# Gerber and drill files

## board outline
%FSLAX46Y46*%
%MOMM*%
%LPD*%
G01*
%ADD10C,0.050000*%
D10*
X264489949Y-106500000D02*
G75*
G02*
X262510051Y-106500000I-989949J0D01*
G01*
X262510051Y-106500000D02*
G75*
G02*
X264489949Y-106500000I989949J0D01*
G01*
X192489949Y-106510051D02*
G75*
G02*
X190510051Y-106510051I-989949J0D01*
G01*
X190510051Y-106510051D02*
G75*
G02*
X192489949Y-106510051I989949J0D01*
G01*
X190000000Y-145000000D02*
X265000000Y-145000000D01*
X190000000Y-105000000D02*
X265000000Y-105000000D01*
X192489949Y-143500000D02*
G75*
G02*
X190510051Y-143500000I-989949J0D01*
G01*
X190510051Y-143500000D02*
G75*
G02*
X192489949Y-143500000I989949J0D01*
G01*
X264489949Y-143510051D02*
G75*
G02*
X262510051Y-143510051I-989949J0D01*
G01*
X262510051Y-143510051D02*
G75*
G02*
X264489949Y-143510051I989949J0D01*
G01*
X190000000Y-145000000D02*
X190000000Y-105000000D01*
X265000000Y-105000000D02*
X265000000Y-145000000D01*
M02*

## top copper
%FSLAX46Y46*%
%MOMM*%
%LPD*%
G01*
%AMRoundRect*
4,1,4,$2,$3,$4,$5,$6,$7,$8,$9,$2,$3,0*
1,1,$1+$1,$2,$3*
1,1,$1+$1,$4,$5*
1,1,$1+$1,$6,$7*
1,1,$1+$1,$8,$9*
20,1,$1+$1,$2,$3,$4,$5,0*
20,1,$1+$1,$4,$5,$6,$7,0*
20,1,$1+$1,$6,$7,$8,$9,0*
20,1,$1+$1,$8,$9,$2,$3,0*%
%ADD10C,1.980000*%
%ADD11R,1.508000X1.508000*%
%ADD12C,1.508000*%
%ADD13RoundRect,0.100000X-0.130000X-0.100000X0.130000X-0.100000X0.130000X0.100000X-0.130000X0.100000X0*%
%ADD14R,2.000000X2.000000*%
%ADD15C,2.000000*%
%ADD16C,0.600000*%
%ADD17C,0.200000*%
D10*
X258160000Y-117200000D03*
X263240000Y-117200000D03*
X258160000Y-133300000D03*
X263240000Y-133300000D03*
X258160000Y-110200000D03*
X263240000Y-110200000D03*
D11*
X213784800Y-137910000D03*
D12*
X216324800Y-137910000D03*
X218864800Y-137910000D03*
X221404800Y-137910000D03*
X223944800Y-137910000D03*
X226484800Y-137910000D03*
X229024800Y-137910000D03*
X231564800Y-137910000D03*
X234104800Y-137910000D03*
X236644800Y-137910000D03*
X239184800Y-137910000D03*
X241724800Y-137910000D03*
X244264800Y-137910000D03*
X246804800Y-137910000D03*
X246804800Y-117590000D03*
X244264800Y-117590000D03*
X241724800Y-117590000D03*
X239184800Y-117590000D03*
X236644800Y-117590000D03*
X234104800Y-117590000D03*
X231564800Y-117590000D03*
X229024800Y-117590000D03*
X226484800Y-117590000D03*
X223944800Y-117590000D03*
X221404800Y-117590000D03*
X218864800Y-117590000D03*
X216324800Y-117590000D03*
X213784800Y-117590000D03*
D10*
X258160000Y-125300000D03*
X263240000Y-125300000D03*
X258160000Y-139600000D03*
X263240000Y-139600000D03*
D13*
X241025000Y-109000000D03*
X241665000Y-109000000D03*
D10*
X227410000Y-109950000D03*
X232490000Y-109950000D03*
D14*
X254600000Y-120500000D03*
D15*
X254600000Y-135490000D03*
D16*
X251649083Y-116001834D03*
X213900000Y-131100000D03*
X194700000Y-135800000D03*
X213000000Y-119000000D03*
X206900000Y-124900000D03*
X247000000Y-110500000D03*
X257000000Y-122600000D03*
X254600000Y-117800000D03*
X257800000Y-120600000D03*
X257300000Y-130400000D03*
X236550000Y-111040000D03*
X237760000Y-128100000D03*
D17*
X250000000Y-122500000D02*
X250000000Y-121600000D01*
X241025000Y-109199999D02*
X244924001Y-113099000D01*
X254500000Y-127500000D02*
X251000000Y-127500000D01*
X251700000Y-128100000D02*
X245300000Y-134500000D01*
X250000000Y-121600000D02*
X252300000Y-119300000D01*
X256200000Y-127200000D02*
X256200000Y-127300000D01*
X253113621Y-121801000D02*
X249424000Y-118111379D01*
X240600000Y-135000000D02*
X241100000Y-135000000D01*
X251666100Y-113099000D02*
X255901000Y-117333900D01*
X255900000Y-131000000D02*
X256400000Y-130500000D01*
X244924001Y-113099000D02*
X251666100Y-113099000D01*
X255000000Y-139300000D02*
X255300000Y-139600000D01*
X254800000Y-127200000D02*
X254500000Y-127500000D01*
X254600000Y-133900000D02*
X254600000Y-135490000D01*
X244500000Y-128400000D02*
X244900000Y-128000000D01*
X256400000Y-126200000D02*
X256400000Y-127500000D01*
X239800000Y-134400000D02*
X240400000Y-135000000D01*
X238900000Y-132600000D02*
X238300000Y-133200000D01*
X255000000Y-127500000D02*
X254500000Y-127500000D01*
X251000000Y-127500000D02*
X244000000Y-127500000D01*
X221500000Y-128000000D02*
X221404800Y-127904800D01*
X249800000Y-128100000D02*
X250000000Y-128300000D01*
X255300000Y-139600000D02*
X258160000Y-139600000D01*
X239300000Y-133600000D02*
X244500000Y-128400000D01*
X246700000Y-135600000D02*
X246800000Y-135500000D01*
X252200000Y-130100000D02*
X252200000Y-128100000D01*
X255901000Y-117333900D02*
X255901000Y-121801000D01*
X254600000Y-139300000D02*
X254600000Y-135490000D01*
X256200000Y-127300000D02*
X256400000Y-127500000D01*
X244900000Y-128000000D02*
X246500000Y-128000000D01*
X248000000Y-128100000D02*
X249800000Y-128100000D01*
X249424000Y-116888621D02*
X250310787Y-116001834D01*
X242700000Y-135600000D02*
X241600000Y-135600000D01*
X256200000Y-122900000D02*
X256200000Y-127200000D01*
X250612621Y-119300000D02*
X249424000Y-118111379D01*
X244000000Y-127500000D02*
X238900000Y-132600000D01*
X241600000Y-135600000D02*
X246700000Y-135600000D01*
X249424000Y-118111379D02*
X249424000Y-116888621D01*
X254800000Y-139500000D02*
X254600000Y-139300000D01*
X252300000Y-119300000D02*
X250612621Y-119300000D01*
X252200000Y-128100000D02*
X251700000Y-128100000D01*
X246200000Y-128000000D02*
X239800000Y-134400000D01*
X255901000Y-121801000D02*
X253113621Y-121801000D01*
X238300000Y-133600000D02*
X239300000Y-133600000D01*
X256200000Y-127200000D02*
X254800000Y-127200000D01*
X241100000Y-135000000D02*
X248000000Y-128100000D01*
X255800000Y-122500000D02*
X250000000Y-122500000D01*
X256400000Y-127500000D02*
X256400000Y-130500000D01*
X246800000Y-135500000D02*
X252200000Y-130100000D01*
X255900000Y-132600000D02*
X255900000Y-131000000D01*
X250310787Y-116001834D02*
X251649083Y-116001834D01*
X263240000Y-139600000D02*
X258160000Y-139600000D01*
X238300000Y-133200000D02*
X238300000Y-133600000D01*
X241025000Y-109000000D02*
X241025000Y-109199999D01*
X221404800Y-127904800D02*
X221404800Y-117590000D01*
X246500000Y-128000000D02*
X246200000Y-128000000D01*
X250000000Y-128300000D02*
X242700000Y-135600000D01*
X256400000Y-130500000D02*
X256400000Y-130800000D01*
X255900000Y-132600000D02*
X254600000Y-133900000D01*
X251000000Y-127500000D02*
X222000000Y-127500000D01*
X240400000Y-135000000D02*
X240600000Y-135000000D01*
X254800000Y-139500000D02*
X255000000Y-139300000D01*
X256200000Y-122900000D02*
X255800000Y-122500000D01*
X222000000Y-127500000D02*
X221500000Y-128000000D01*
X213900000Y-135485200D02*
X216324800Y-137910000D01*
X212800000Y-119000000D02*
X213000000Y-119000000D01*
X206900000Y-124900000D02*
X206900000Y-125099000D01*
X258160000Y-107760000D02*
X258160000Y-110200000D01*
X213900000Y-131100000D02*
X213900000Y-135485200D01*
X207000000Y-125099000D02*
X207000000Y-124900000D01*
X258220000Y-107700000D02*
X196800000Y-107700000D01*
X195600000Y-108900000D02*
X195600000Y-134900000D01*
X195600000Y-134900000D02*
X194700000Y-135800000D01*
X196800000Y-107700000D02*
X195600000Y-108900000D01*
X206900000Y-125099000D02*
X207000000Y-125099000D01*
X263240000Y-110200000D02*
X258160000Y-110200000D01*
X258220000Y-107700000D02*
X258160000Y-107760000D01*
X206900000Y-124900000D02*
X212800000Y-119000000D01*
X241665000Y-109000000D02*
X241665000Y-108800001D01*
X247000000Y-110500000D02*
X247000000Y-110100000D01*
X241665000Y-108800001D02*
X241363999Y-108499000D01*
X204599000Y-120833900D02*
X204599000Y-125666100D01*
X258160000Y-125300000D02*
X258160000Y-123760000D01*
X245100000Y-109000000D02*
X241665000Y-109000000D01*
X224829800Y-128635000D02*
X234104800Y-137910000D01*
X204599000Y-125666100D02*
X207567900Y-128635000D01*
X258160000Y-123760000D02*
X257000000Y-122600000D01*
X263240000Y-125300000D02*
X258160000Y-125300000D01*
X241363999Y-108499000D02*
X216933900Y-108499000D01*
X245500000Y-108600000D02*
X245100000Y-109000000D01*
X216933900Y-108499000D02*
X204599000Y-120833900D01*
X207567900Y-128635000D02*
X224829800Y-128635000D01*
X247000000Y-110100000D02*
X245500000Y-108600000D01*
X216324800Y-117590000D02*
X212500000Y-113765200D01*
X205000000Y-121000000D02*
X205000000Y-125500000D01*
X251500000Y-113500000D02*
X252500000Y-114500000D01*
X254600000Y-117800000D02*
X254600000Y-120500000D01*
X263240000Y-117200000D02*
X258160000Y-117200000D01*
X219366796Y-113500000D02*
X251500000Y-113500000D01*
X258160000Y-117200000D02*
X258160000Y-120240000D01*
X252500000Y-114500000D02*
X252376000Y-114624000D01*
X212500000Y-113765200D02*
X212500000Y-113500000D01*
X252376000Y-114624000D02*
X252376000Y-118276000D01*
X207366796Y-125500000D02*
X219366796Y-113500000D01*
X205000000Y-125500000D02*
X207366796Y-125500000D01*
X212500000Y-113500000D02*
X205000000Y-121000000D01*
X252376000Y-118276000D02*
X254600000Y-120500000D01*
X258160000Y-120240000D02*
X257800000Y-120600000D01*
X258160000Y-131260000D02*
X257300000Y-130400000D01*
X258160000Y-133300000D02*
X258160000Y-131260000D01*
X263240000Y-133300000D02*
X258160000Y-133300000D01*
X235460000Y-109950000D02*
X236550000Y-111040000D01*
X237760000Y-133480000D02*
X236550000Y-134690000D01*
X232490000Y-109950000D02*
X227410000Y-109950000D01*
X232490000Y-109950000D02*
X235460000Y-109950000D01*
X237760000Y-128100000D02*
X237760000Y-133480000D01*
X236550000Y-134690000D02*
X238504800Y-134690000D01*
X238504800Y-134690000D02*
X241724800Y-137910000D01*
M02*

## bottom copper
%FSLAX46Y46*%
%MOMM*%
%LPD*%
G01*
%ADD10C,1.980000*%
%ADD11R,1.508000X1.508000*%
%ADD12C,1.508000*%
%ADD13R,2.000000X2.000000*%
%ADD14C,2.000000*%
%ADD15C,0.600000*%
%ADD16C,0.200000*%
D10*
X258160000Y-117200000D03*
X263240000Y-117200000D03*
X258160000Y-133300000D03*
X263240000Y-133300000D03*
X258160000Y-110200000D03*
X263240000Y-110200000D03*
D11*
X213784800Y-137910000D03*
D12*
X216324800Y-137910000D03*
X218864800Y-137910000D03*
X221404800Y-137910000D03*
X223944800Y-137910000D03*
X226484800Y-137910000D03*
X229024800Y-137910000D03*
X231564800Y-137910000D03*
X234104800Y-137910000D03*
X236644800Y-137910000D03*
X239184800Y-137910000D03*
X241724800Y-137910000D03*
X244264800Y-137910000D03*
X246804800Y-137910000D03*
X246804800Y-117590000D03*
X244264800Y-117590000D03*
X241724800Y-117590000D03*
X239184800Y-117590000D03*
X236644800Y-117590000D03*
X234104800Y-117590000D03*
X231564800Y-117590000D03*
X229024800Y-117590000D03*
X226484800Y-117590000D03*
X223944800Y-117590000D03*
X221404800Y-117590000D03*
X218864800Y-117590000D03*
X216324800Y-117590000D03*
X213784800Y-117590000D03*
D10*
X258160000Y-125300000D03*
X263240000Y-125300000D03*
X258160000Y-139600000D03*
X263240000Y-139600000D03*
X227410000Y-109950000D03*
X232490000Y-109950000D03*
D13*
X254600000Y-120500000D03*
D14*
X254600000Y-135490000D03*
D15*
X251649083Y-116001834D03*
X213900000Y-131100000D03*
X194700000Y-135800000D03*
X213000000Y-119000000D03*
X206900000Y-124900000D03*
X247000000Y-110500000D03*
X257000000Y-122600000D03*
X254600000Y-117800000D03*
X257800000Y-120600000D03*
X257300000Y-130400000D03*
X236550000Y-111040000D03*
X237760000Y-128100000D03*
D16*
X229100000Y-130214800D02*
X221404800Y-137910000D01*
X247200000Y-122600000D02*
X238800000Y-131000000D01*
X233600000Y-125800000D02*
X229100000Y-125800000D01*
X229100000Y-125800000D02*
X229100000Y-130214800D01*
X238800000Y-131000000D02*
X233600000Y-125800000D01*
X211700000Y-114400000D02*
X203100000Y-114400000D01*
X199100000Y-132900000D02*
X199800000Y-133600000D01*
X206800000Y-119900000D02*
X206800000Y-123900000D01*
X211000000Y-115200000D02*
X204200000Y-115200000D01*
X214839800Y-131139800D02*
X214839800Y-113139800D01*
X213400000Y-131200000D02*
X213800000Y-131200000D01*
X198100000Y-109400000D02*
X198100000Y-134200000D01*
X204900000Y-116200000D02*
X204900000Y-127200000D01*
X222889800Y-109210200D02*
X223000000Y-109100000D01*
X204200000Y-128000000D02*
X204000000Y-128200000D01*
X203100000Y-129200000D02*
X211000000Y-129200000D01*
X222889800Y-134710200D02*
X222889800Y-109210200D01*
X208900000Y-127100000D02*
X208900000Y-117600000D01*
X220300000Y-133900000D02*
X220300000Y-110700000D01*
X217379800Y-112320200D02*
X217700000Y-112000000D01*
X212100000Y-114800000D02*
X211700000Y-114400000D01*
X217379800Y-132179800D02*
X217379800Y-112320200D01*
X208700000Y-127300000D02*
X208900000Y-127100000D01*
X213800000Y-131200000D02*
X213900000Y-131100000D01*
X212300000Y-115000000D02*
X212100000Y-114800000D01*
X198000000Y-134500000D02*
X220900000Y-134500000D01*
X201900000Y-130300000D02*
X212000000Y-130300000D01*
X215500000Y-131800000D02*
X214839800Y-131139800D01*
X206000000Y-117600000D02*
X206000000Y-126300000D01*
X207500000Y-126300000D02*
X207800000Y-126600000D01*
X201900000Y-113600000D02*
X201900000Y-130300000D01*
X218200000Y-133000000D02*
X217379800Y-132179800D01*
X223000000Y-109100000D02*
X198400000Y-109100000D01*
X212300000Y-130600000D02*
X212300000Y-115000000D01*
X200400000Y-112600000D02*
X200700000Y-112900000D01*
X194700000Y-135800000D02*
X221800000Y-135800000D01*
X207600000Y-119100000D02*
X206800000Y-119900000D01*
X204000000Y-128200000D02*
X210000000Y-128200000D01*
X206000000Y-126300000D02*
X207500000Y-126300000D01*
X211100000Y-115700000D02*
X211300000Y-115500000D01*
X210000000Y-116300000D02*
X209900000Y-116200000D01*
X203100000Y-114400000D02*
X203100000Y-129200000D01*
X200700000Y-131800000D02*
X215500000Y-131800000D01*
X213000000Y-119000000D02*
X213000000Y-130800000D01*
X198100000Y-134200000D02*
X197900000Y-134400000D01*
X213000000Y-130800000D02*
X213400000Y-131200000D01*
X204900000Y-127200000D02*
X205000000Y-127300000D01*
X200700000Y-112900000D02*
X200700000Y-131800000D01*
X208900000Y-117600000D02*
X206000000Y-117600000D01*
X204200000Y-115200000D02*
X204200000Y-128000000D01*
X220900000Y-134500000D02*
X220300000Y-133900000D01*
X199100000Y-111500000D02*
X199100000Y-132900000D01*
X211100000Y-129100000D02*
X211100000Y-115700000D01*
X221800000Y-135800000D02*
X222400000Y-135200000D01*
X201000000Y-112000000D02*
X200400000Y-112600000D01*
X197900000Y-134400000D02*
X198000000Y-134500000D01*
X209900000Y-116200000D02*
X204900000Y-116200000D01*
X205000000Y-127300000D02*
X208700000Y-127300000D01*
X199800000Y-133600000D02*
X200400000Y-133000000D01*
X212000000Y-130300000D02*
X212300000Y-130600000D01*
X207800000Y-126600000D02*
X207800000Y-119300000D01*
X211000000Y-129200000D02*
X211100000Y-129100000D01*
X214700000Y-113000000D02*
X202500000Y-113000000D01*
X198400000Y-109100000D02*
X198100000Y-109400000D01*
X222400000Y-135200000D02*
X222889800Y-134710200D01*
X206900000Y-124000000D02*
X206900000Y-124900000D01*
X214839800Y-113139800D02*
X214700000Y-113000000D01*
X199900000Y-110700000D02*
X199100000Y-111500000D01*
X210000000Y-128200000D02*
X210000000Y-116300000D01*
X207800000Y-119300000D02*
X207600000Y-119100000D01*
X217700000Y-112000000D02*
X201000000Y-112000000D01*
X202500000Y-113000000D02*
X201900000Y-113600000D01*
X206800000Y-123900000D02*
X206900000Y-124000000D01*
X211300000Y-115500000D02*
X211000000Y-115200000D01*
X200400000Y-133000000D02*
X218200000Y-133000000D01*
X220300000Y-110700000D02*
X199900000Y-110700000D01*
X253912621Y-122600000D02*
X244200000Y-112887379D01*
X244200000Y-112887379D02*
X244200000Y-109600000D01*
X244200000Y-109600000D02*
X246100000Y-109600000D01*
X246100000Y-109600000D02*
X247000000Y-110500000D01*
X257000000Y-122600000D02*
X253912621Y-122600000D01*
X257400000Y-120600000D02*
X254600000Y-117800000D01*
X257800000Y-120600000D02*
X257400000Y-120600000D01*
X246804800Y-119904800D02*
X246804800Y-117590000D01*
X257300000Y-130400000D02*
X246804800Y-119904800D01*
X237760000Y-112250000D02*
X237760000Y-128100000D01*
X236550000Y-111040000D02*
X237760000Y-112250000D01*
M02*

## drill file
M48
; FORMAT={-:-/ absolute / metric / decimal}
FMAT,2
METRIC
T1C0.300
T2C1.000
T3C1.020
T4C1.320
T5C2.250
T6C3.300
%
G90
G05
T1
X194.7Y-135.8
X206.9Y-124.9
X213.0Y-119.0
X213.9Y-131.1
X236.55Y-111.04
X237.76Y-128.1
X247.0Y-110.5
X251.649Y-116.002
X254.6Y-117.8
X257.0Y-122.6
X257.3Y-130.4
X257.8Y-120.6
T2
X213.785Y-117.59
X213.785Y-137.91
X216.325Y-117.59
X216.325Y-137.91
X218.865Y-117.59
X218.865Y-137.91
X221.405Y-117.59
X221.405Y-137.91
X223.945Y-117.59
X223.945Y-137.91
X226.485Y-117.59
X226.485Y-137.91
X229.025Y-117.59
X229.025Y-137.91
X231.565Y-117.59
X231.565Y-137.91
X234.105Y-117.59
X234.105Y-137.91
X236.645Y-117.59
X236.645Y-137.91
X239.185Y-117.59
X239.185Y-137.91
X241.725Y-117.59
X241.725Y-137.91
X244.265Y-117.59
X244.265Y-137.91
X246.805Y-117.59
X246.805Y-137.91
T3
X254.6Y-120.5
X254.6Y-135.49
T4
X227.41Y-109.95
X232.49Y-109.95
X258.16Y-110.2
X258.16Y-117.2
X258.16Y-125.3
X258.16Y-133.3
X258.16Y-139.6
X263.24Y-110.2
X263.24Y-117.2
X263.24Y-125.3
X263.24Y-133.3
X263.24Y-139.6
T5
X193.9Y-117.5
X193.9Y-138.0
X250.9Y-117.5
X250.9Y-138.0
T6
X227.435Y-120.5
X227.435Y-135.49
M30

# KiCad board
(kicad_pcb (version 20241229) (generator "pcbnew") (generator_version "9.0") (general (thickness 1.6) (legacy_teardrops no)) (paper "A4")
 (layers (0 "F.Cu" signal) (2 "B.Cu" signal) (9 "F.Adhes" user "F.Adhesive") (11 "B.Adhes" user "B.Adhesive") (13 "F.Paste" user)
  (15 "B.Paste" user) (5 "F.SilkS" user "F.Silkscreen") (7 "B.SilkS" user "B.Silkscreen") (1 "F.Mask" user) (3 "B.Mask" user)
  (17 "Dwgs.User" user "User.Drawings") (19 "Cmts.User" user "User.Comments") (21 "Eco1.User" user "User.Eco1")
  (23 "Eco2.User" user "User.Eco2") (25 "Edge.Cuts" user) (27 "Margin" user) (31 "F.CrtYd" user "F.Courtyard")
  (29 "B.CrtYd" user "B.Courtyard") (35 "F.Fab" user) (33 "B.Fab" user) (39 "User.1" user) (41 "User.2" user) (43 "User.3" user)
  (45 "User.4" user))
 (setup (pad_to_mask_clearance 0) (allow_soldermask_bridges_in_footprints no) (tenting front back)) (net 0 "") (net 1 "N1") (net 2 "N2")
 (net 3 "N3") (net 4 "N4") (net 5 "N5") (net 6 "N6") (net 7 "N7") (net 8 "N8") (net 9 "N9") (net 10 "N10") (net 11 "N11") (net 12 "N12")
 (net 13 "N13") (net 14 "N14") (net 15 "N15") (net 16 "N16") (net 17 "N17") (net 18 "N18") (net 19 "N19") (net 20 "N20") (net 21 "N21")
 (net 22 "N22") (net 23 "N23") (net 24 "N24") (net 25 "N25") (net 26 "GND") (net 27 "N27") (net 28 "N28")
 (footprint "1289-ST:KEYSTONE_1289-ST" (layer "F.Cu") (at 260.7 117.2)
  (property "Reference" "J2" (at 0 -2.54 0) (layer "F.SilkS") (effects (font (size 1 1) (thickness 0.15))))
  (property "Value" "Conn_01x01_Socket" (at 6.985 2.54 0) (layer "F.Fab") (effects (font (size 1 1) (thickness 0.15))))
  (pad "1_1" thru_hole circle (at -2.54 0) (size 1.98 1.98) (drill 1.32) (layers "*.Cu" "*.Mask") (remove_unused_layers no) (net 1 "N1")
   (solder_mask_margin 0.102))
  (pad "1_2" thru_hole circle (at 2.54 0) (size 1.98 1.98) (drill 1.32) (layers "*.Cu" "*.Mask") (remove_unused_layers no) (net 1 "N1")
   (solder_mask_margin 0.102)))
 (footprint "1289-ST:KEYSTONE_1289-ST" (layer "F.Cu") (at 260.7 133.3)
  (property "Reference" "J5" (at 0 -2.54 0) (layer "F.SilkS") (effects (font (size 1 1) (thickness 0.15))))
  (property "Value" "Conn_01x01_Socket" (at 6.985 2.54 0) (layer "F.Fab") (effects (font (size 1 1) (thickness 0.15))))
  (pad "1_1" thru_hole circle (at -2.54 0) (size 1.98 1.98) (drill 1.32) (layers "*.Cu" "*.Mask") (remove_unused_layers no) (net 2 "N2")
   (solder_mask_margin 0.102))
  (pad "1_2" thru_hole circle (at 2.54 0) (size 1.98 1.98) (drill 1.32) (layers "*.Cu" "*.Mask") (remove_unused_layers no) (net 2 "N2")
   (solder_mask_margin 0.102)))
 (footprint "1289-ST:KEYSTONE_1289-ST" (layer "F.Cu") (at 260.7 110.2)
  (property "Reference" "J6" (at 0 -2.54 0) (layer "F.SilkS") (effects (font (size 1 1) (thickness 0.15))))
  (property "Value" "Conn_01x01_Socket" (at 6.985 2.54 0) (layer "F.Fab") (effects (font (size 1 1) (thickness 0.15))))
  (pad "1_1" thru_hole circle (at -2.54 0) (size 1.98 1.98) (drill 1.32) (layers "*.Cu" "*.Mask") (remove_unused_layers no) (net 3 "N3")
   (solder_mask_margin 0.102))
  (pad "1_2" thru_hole circle (at 2.54 0) (size 1.98 1.98) (drill 1.32) (layers "*.Cu" "*.Mask") (remove_unused_layers no) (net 3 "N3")
   (solder_mask_margin 0.102)))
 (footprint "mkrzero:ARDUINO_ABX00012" (layer "F.Cu") (at 191.65 140.25)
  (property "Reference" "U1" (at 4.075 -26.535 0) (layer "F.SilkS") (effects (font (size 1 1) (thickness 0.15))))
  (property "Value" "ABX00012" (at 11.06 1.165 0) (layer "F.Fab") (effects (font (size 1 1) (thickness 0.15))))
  (pad "" np_thru_hole circle (at 2.25 -22.75) (size 2.25 2.25) (drill 2.25) (layers "*.Cu" "*.Mask"))
  (pad "" np_thru_hole circle (at 2.25 -2.25) (size 2.25 2.25) (drill 2.25) (layers "*.Cu" "*.Mask"))
  (pad "" np_thru_hole circle (at 59.25 -22.75) (size 2.25 2.25) (drill 2.25) (layers "*.Cu" "*.Mask"))
  (pad "" np_thru_hole circle (at 59.25 -2.25) (size 2.25 2.25) (drill 2.25) (layers "*.Cu" "*.Mask"))
  (pad "1" thru_hole rect (at 22.1348 -2.34) (size 1.508 1.508) (drill 1) (layers "*.Cu" "*.Mask") (remove_unused_layers no) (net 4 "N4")
   (solder_mask_margin 0.102))
  (pad "2" thru_hole circle (at 24.6748 -2.34) (size 1.508 1.508) (drill 1) (layers "*.Cu" "*.Mask") (remove_unused_layers no) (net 3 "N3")
   (solder_mask_margin 0.102))
  (pad "3" thru_hole circle (at 27.2148 -2.34) (size 1.508 1.508) (drill 1) (layers "*.Cu" "*.Mask") (remove_unused_layers no) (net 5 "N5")
   (solder_mask_margin 0.102))
  (pad "4" thru_hole circle (at 29.7548 -2.34) (size 1.508 1.508) (drill 1) (layers "*.Cu" "*.Mask") (remove_unused_layers no) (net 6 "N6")
   (solder_mask_margin 0.102))
  (pad "5" thru_hole circle (at 32.2948 -2.34) (size 1.508 1.508) (drill 1) (layers "*.Cu" "*.Mask") (remove_unused_layers no) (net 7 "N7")
   (solder_mask_margin 0.102))
  (pad "6" thru_hole circle (at 34.8348 -2.34) (size 1.508 1.508) (drill 1) (layers "*.Cu" "*.Mask") (remove_unused_layers no) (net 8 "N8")
   (solder_mask_margin 0.102))
  (pad "7" thru_hole circle (at 37.3748 -2.34) (size 1.508 1.508) (drill 1) (layers "*.Cu" "*.Mask") (remove_unused_layers no) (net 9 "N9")
   (solder_mask_margin 0.102))
  (pad "8" thru_hole circle (at 39.9148 -2.34) (size 1.508 1.508) (drill 1) (layers "*.Cu" "*.Mask") (remove_unused_layers no)
   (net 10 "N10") (solder_mask_margin 0.102))
  (pad "9" thru_hole circle (at 42.4548 -2.34) (size 1.508 1.508) (drill 1) (layers "*.Cu" "*.Mask") (remove_unused_layers no)
   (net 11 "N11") (solder_mask_margin 0.102))
  (pad "10" thru_hole circle (at 44.9948 -2.34) (size 1.508 1.508) (drill 1) (layers "*.Cu" "*.Mask") (remove_unused_layers no)
   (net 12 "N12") (solder_mask_margin 0.102))
  (pad "11" thru_hole circle (at 47.5348 -2.34) (size 1.508 1.508) (drill 1) (layers "*.Cu" "*.Mask") (remove_unused_layers no)
   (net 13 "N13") (solder_mask_margin 0.102))
  (pad "12" thru_hole circle (at 50.0748 -2.34) (size 1.508 1.508) (drill 1) (layers "*.Cu" "*.Mask") (remove_unused_layers no)
   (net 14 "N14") (solder_mask_margin 0.102))
  (pad "13" thru_hole circle (at 52.6148 -2.34) (size 1.508 1.508) (drill 1) (layers "*.Cu" "*.Mask") (remove_unused_layers no)
   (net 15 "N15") (solder_mask_margin 0.102))
  (pad "14" thru_hole circle (at 55.1548 -2.34) (size 1.508 1.508) (drill 1) (layers "*.Cu" "*.Mask") (remove_unused_layers no)
   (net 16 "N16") (solder_mask_margin 0.102))
  (pad "15" thru_hole circle (at 55.1548 -22.66) (size 1.508 1.508) (drill 1) (layers "*.Cu" "*.Mask") (remove_unused_layers no)
   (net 2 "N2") (solder_mask_margin 0.102))
  (pad "16" thru_hole circle (at 52.6148 -22.66) (size 1.508 1.508) (drill 1) (layers "*.Cu" "*.Mask") (remove_unused_layers no)
   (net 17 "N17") (solder_mask_margin 0.102))
  (pad "17" thru_hole circle (at 50.0748 -22.66) (size 1.508 1.508) (drill 1) (layers "*.Cu" "*.Mask") (remove_unused_layers no)
   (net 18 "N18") (solder_mask_margin 0.102))
  (pad "18" thru_hole circle (at 47.5348 -22.66) (size 1.508 1.508) (drill 1) (layers "*.Cu" "*.Mask") (remove_unused_layers no)
   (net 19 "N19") (solder_mask_margin 0.102))
  (pad "19" thru_hole circle (at 44.9948 -22.66) (size 1.508 1.508) (drill 1) (layers "*.Cu" "*.Mask") (remove_unused_layers no)
   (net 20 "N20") (solder_mask_margin 0.102))
  (pad "20" thru_hole circle (at 42.4548 -22.66) (size 1.508 1.508) (drill 1) (layers "*.Cu" "*.Mask") (remove_unused_layers no)
   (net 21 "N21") (solder_mask_margin 0.102))
  (pad "21" thru_hole circle (at 39.9148 -22.66) (size 1.508 1.508) (drill 1) (layers "*.Cu" "*.Mask") (remove_unused_layers no)
   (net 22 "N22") (solder_mask_margin 0.102))
  (pad "22" thru_hole circle (at 37.3748 -22.66) (size 1.508 1.508) (drill 1) (layers "*.Cu" "*.Mask") (remove_unused_layers no)
   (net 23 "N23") (solder_mask_margin 0.102))
  (pad "23" thru_hole circle (at 34.8348 -22.66) (size 1.508 1.508) (drill 1) (layers "*.Cu" "*.Mask") (remove_unused_layers no)
   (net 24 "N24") (solder_mask_margin 0.102))
  (pad "24" thru_hole circle (at 32.2948 -22.66) (size 1.508 1.508) (drill 1) (layers "*.Cu" "*.Mask") (remove_unused_layers no)
   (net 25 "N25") (solder_mask_margin 0.102))
  (pad "25" thru_hole circle (at 29.7548 -22.66) (size 1.508 1.508) (drill 1) (layers "*.Cu" "*.Mask") (remove_unused_layers no)
   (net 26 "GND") (solder_mask_margin 0.102))
  (pad "26" thru_hole circle (at 27.2148 -22.66) (size 1.508 1.508) (drill 1) (layers "*.Cu" "*.Mask") (remove_unused_layers no)
   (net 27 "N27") (solder_mask_margin 0.102))
  (pad "27" thru_hole circle (at 24.6748 -22.66) (size 1.508 1.508) (drill 1) (layers "*.Cu" "*.Mask") (remove_unused_layers no)
   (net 1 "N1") (solder_mask_margin 0.102))
  (pad "28" thru_hole circle (at 22.1348 -22.66) (size 1.508 1.508) (drill 1) (layers "*.Cu" "*.Mask") (remove_unused_layers no)
   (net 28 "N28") (solder_mask_margin 0.102)))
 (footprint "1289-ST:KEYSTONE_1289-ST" (layer "F.Cu") (at 260.7 125.3)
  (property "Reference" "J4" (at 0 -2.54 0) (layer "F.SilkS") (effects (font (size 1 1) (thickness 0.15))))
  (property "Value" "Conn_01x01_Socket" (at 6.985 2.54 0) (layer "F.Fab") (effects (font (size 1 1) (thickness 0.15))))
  (pad "1_1" thru_hole circle (at -2.54 0) (size 1.98 1.98) (drill 1.32) (layers "*.Cu" "*.Mask") (remove_unused_layers no) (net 11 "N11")
   (solder_mask_margin 0.102))
  (pad "1_2" thru_hole circle (at 2.54 0) (size 1.98 1.98) (drill 1.32) (layers "*.Cu" "*.Mask") (remove_unused_layers no) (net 11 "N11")
   (solder_mask_margin 0.102)))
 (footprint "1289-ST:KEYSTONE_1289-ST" (layer "F.Cu") (at 260.7 139.6)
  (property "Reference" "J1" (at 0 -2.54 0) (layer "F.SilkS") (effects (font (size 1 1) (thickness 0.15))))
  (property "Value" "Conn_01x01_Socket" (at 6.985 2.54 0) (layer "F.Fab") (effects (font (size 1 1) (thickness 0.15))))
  (pad "1_1" thru_hole circle (at -2.54 0) (size 1.98 1.98) (drill 1.32) (layers "*.Cu" "*.Mask") (remove_unused_layers no) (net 26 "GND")
   (solder_mask_margin 0.102))
  (pad "1_2" thru_hole circle (at 2.54 0) (size 1.98 1.98) (drill 1.32) (layers "*.Cu" "*.Mask") (remove_unused_layers no) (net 26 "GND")
   (solder_mask_margin 0.102)))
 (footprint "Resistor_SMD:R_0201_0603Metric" (layer "F.Cu") (at 241.345 109)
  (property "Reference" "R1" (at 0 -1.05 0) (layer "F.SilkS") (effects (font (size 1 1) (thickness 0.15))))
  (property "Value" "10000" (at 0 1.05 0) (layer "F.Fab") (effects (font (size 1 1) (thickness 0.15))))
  (pad "" smd roundrect (at -0.345 0) (size 0.318 0.36) (layers "F.Paste") (roundrect_rratio 0.25))
  (pad "" smd roundrect (at 0.345 0) (size 0.318 0.36) (layers "F.Paste") (roundrect_rratio 0.25))
  (pad "1" smd roundrect (at -0.32 0) (size 0.46 0.4) (layers "F.Cu" "F.Mask") (roundrect_rratio 0.25) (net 26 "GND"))
  (pad "2" smd roundrect (at 0.32 0) (size 0.46 0.4) (layers "F.Cu" "F.Mask") (roundrect_rratio 0.25) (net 11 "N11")))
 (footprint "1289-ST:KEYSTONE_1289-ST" (layer "F.Cu") (at 229.95 109.95)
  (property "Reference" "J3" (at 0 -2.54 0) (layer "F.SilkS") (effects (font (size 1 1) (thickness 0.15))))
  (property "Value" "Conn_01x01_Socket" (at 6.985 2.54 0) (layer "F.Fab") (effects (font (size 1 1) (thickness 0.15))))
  (pad "1_1" thru_hole circle (at -2.54 0) (size 1.98 1.98) (drill 1.32) (layers "*.Cu" "*.Mask") (remove_unused_layers no) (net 14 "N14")
   (solder_mask_margin 0.102))
  (pad "1_2" thru_hole circle (at 2.54 0) (size 1.98 1.98) (drill 1.32) (layers "*.Cu" "*.Mask") (remove_unused_layers no) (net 14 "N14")
   (solder_mask_margin 0.102)))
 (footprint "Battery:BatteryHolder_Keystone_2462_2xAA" (layer "B.Cu") (at 254.6 120.5 180)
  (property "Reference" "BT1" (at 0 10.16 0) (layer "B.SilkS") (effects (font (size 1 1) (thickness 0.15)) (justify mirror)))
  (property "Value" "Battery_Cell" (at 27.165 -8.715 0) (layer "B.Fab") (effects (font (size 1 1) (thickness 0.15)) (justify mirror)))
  (pad "" np_thru_hole circle (at 27.165 -14.99 180) (size 3.3 3.3) (drill 3.3) (layers "*.Cu" "*.Mask"))
  (pad "" np_thru_hole circle (at 27.165 0 180) (size 3.3 3.3) (drill 3.3) (layers "*.Cu" "*.Mask"))
  (pad "1" thru_hole rect (at 0 0 180) (size 2 2) (drill 1.02) (layers "*.Cu" "*.Mask") (remove_unused_layers no) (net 1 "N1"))
  (pad "2" thru_hole circle (at 0 -14.99 180) (size 2 2) (drill 1.02) (layers "*.Cu" "*.Mask") (remove_unused_layers no) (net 26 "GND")))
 (gr_circle (center 263.5 106.5) (end 264.2 105.8) (stroke (width 0.05) (type default)) (fill no) (layer "Edge.Cuts"))
 (gr_circle (center 191.5 106.510051) (end 192.2 105.810051) (stroke (width 0.05) (type default)) (fill no) (layer "Edge.Cuts"))
 (gr_line (start 190 145) (end 265 145) (stroke (width 0.05) (type default)) (layer "Edge.Cuts"))
 (gr_line (start 190 105) (end 265 105) (stroke (width 0.05) (type default)) (layer "Edge.Cuts"))
 (gr_circle (center 191.5 143.5) (end 192.2 142.8) (stroke (width 0.05) (type default)) (fill no) (layer "Edge.Cuts"))
 (gr_circle (center 263.5 143.510051) (end 264.2 142.810051) (stroke (width 0.05) (type default)) (fill no) (layer "Edge.Cuts"))
 (gr_line (start 190 145) (end 190 105) (stroke (width 0.05) (type default)) (layer "Edge.Cuts"))
 (gr_line (start 265 105) (end 265 145) (stroke (width 0.05) (type default)) (layer "Edge.Cuts"))
 (segment (start 250 122.5) (end 250 121.6) (width 0.2) (layer "F.Cu") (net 26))
 (segment (start 241.025 109.199999) (end 244.924001 113.099) (width 0.2) (layer "F.Cu") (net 26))
 (segment (start 254.5 127.5) (end 251 127.5) (width 0.2) (layer "F.Cu") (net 26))
 (segment (start 251.7 128.1) (end 245.3 134.5) (width 0.2) (layer "F.Cu") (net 26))
 (segment (start 250 121.6) (end 252.3 119.3) (width 0.2) (layer "F.Cu") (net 26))
 (segment (start 256.2 127.2) (end 256.2 127.3) (width 0.2) (layer "F.Cu") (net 26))
 (segment (start 253.113621 121.801) (end 249.424 118.111379) (width 0.2) (layer "F.Cu") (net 26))
 (segment (start 240.6 135) (end 241.1 135) (width 0.2) (layer "F.Cu") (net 26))
 (segment (start 251.6661 113.099) (end 255.901 117.3339) (width 0.2) (layer "F.Cu") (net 26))
 (segment (start 255.9 131) (end 256.4 130.5) (width 0.2) (layer "F.Cu") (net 26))
 (segment (start 244.924001 113.099) (end 251.6661 113.099) (width 0.2) (layer "F.Cu") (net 26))
 (segment (start 255 139.3) (end 255.3 139.6) (width 0.2) (layer "F.Cu") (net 26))
 (segment (start 254.8 127.2) (end 254.5 127.5) (width 0.2) (layer "F.Cu") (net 26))
 (segment (start 254.6 133.9) (end 254.6 135.49) (width 0.2) (layer "F.Cu") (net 26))
 (segment (start 244.5 128.4) (end 244.9 128) (width 0.2) (layer "F.Cu") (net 26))
 (segment (start 256.4 126.2) (end 256.4 127.5) (width 0.2) (layer "F.Cu") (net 26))
 (segment (start 239.8 134.4) (end 240.4 135) (width 0.2) (layer "F.Cu") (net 26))
 (segment (start 238.9 132.6) (end 238.3 133.2) (width 0.2) (layer "F.Cu") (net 26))
 (segment (start 255 127.5) (end 254.5 127.5) (width 0.2) (layer "F.Cu") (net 26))
 (segment (start 251 127.5) (end 244 127.5) (width 0.2) (layer "F.Cu") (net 26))
 (segment (start 221.5 128) (end 221.4048 127.9048) (width 0.2) (layer "F.Cu") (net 26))
 (segment (start 249.8 128.1) (end 250 128.3) (width 0.2) (layer "F.Cu") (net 26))
 (segment (start 255.3 139.6) (end 258.16 139.6) (width 0.2) (layer "F.Cu") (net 26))
 (segment (start 239.3 133.6) (end 244.5 128.4) (width 0.2) (layer "F.Cu") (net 26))
 (segment (start 246.7 135.6) (end 246.8 135.5) (width 0.2) (layer "F.Cu") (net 26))
 (segment (start 252.2 130.1) (end 252.2 128.1) (width 0.2) (layer "F.Cu") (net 26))
 (segment (start 255.901 117.3339) (end 255.901 121.801) (width 0.2) (layer "F.Cu") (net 26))
 (segment (start 254.6 139.3) (end 254.6 135.49) (width 0.2) (layer "F.Cu") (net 26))
 (segment (start 256.2 127.3) (end 256.4 127.5) (width 0.2) (layer "F.Cu") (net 26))
 (segment (start 244.9 128) (end 246.5 128) (width 0.2) (layer "F.Cu") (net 26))
 (segment (start 248 128.1) (end 249.8 128.1) (width 0.2) (layer "F.Cu") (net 26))
 (segment (start 249.424 116.888621) (end 250.310787 116.001834) (width 0.2) (layer "F.Cu") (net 26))
 (segment (start 242.7 135.6) (end 241.6 135.6) (width 0.2) (layer "F.Cu") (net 26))
 (segment (start 256.2 122.9) (end 256.2 127.2) (width 0.2) (layer "F.Cu") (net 26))
 (segment (start 250.612621 119.3) (end 249.424 118.111379) (width 0.2) (layer "F.Cu") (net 26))
 (segment (start 244 127.5) (end 238.9 132.6) (width 0.2) (layer "F.Cu") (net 26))
 (segment (start 241.6 135.6) (end 246.7 135.6) (width 0.2) (layer "F.Cu") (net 26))
 (segment (start 249.424 118.111379) (end 249.424 116.888621) (width 0.2) (layer "F.Cu") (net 26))
 (segment (start 254.8 139.5) (end 254.6 139.3) (width 0.2) (layer "F.Cu") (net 26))
 (segment (start 252.3 119.3) (end 250.612621 119.3) (width 0.2) (layer "F.Cu") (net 26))
 (segment (start 252.2 128.1) (end 251.7 128.1) (width 0.2) (layer "F.Cu") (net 26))
 (segment (start 246.2 128) (end 239.8 134.4) (width 0.2) (layer "F.Cu") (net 26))
 (segment (start 255.901 121.801) (end 253.113621 121.801) (width 0.2) (layer "F.Cu") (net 26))
 (segment (start 238.3 133.6) (end 239.3 133.6) (width 0.2) (layer "F.Cu") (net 26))
 (segment (start 256.2 127.2) (end 254.8 127.2) (width 0.2) (layer "F.Cu") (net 26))
 (segment (start 241.1 135) (end 248 128.1) (width 0.2) (layer "F.Cu") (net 26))
 (segment (start 255.8 122.5) (end 250 122.5) (width 0.2) (layer "F.Cu") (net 26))
 (segment (start 256.4 127.5) (end 256.4 130.5) (width 0.2) (layer "F.Cu") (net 26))
 (segment (start 246.8 135.5) (end 252.2 130.1) (width 0.2) (layer "F.Cu") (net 26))
 (segment (start 255.9 132.6) (end 255.9 131) (width 0.2) (layer "F.Cu") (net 26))
 (segment (start 250.310787 116.001834) (end 251.649083 116.001834) (width 0.2) (layer "F.Cu") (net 26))
 (segment (start 263.24 139.6) (end 258.16 139.6) (width 0.2) (layer "F.Cu") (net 26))
 (segment (start 238.3 133.2) (end 238.3 133.6) (width 0.2) (layer "F.Cu") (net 26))
 (segment (start 241.025 109) (end 241.025 109.199999) (width 0.2) (layer "F.Cu") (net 26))
 (segment (start 221.4048 127.9048) (end 221.4048 117.59) (width 0.2) (layer "F.Cu") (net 26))
 (segment (start 246.5 128) (end 246.2 128) (width 0.2) (layer "F.Cu") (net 26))
 (segment (start 250 128.3) (end 242.7 135.6) (width 0.2) (layer "F.Cu") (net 26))
 (segment (start 256.4 130.5) (end 256.4 130.8) (width 0.2) (layer "F.Cu") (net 26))
 (segment (start 255.9 132.6) (end 254.6 133.9) (width 0.2) (layer "F.Cu") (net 26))
 (segment (start 251 127.5) (end 222 127.5) (width 0.2) (layer "F.Cu") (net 26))
 (segment (start 240.4 135) (end 240.6 135) (width 0.2) (layer "F.Cu") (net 26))
 (segment (start 254.8 139.5) (end 255 139.3) (width 0.2) (layer "F.Cu") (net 26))
 (segment (start 256.2 122.9) (end 255.8 122.5) (width 0.2) (layer "F.Cu") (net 26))
 (segment (start 222 127.5) (end 221.5 128) (width 0.2) (layer "F.Cu") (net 26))
 (via (at 251.649083 116.001834) (size 0.6) (drill 0.3) (layers "F.Cu" "B.Cu") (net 26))
 (segment (start 229.1 130.2148) (end 221.4048 137.91) (width 0.2) (layer "B.Cu") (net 6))
 (segment (start 247.2 122.6) (end 238.8 131) (width 0.2) (layer "B.Cu") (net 6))
 (segment (start 233.6 125.8) (end 229.1 125.8) (width 0.2) (layer "B.Cu") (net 6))
 (segment (start 229.1 125.8) (end 229.1 130.2148) (width 0.2) (layer "B.Cu") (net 6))
 (segment (start 238.8 131) (end 233.6 125.8) (width 0.2) (layer "B.Cu") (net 6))
 (segment (start 213.9 135.4852) (end 216.3248 137.91) (width 0.2) (layer "F.Cu") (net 3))
 (segment (start 212.8 119) (end 213 119) (width 0.2) (layer "F.Cu") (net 3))
 (segment (start 206.9 124.9) (end 206.9 125.099) (width 0.2) (layer "F.Cu") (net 3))
 (segment (start 258.16 107.76) (end 258.16 110.2) (width 0.2) (layer "F.Cu") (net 3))
 (segment (start 213.9 131.1) (end 213.9 135.4852) (width 0.2) (layer "F.Cu") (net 3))
 (segment (start 207 125.099) (end 207 124.9) (width 0.2) (layer "F.Cu") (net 3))
 (segment (start 258.22 107.7) (end 196.8 107.7) (width 0.2) (layer "F.Cu") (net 3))
 (segment (start 195.6 108.9) (end 195.6 134.9) (width 0.2) (layer "F.Cu") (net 3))
 (segment (start 195.6 134.9) (end 194.7 135.8) (width 0.2) (layer "F.Cu") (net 3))
 (segment (start 196.8 107.7) (end 195.6 108.9) (width 0.2) (layer "F.Cu") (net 3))
 (segment (start 206.9 125.099) (end 207 125.099) (width 0.2) (layer "F.Cu") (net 3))
 (segment (start 263.24 110.2) (end 258.16 110.2) (width 0.2) (layer "F.Cu") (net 3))
 (segment (start 258.22 107.7) (end 258.16 107.76) (width 0.2) (layer "F.Cu") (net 3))
 (segment (start 206.9 124.9) (end 212.8 119) (width 0.2) (layer "F.Cu") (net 3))
 (via (at 213.9 131.1) (size 0.6) (drill 0.3) (layers "F.Cu" "B.Cu") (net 3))
 (via (at 194.7 135.8) (size 0.6) (drill 0.3) (layers "F.Cu" "B.Cu") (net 3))
 (via (at 213 119) (size 0.6) (drill 0.3) (layers "F.Cu" "B.Cu") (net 3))
 (via (at 206.9 124.9) (size 0.6) (drill 0.3) (layers "F.Cu" "B.Cu") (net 3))
 (segment (start 211.7 114.4) (end 203.1 114.4) (width 0.2) (layer "B.Cu") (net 3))
 (segment (start 199.1 132.9) (end 199.8 133.6) (width 0.2) (layer "B.Cu") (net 3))
 (segment (start 206.8 119.9) (end 206.8 123.9) (width 0.2) (layer "B.Cu") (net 3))
 (segment (start 211 115.2) (end 204.2 115.2) (width 0.2) (layer "B.Cu") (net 3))
 (segment (start 214.8398 131.1398) (end 214.8398 113.1398) (width 0.2) (layer "B.Cu") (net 3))
 (segment (start 213.4 131.2) (end 213.8 131.2) (width 0.2) (layer "B.Cu") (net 3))
 (segment (start 198.1 109.4) (end 198.1 134.2) (width 0.2) (layer "B.Cu") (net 3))
 (segment (start 204.9 116.2) (end 204.9 127.2) (width 0.2) (layer "B.Cu") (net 3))
 (segment (start 222.8898 109.2102) (end 223 109.1) (width 0.2) (layer "B.Cu") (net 3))
 (segment (start 204.2 128) (end 204 128.2) (width 0.2) (layer "B.Cu") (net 3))
 (segment (start 203.1 129.2) (end 211 129.2) (width 0.2) (layer "B.Cu") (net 3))
 (segment (start 222.8898 134.7102) (end 222.8898 109.2102) (width 0.2) (layer "B.Cu") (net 3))
 (segment (start 208.9 127.1) (end 208.9 117.6) (width 0.2) (layer "B.Cu") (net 3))
 (segment (start 220.3 133.9) (end 220.3 110.7) (width 0.2) (layer "B.Cu") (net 3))
 (segment (start 217.3798 112.3202) (end 217.7 112) (width 0.2) (layer "B.Cu") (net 3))
 (segment (start 212.1 114.8) (end 211.7 114.4) (width 0.2) (layer "B.Cu") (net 3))
 (segment (start 217.3798 132.1798) (end 217.3798 112.3202) (width 0.2) (layer "B.Cu") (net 3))
 (segment (start 208.7 127.3) (end 208.9 127.1) (width 0.2) (layer "B.Cu") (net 3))
 (segment (start 213.8 131.2) (end 213.9 131.1) (width 0.2) (layer "B.Cu") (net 3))
 (segment (start 212.3 115) (end 212.1 114.8) (width 0.2) (layer "B.Cu") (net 3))
 (segment (start 198 134.5) (end 220.9 134.5) (width 0.2) (layer "B.Cu") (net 3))
 (segment (start 201.9 130.3) (end 212 130.3) (width 0.2) (layer "B.Cu") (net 3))
 (segment (start 215.5 131.8) (end 214.8398 131.1398) (width 0.2) (layer "B.Cu") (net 3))
 (segment (start 206 117.6) (end 206 126.3) (width 0.2) (layer "B.Cu") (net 3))
 (segment (start 207.5 126.3) (end 207.8 126.6) (width 0.2) (layer "B.Cu") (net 3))
 (segment (start 201.9 113.6) (end 201.9 130.3) (width 0.2) (layer "B.Cu") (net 3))
 (segment (start 218.2 133) (end 217.3798 132.1798) (width 0.2) (layer "B.Cu") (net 3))
 (segment (start 223 109.1) (end 198.4 109.1) (width 0.2) (layer "B.Cu") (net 3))
 (segment (start 212.3 130.6) (end 212.3 115) (width 0.2) (layer "B.Cu") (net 3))
 (segment (start 200.4 112.6) (end 200.7 112.9) (width 0.2) (layer "B.Cu") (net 3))
 (segment (start 194.7 135.8) (end 221.8 135.8) (width 0.2) (layer "B.Cu") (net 3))
 (segment (start 207.6 119.1) (end 206.8 119.9) (width 0.2) (layer "B.Cu") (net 3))
 (segment (start 204 128.2) (end 210 128.2) (width 0.2) (layer "B.Cu") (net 3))
 (segment (start 206 126.3) (end 207.5 126.3) (width 0.2) (layer "B.Cu") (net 3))
 (segment (start 211.1 115.7) (end 211.3 115.5) (width 0.2) (layer "B.Cu") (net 3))
 (segment (start 210 116.3) (end 209.9 116.2) (width 0.2) (layer "B.Cu") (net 3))
 (segment (start 203.1 114.4) (end 203.1 129.2) (width 0.2) (layer "B.Cu") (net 3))
 (segment (start 200.7 131.8) (end 215.5 131.8) (width 0.2) (layer "B.Cu") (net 3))
 (segment (start 213 119) (end 213 130.8) (width 0.2) (layer "B.Cu") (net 3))
 (segment (start 198.1 134.2) (end 197.9 134.4) (width 0.2) (layer "B.Cu") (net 3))
 (segment (start 213 130.8) (end 213.4 131.2) (width 0.2) (layer "B.Cu") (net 3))
 (segment (start 204.9 127.2) (end 205 127.3) (width 0.2) (layer "B.Cu") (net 3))
 (segment (start 200.7 112.9) (end 200.7 131.8) (width 0.2) (layer "B.Cu") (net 3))
 (segment (start 208.9 117.6) (end 206 117.6) (width 0.2) (layer "B.Cu") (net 3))
 (segment (start 204.2 115.2) (end 204.2 128) (width 0.2) (layer "B.Cu") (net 3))
 (segment (start 220.9 134.5) (end 220.3 133.9) (width 0.2) (layer "B.Cu") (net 3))
 (segment (start 199.1 111.5) (end 199.1 132.9) (width 0.2) (layer "B.Cu") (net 3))
 (segment (start 211.1 129.1) (end 211.1 115.7) (width 0.2) (layer "B.Cu") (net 3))
 (segment (start 221.8 135.8) (end 222.4 135.2) (width 0.2) (layer "B.Cu") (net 3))
 (segment (start 201 112) (end 200.4 112.6) (width 0.2) (layer "B.Cu") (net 3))
 (segment (start 197.9 134.4) (end 198 134.5) (width 0.2) (layer "B.Cu") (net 3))
 (segment (start 209.9 116.2) (end 204.9 116.2) (width 0.2) (layer "B.Cu") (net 3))
 (segment (start 205 127.3) (end 208.7 127.3) (width 0.2) (layer "B.Cu") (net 3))
 (segment (start 199.8 133.6) (end 200.4 133) (width 0.2) (layer "B.Cu") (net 3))
 (segment (start 212 130.3) (end 212.3 130.6) (width 0.2) (layer "B.Cu") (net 3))
 (segment (start 207.8 126.6) (end 207.8 119.3) (width 0.2) (layer "B.Cu") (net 3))
 (segment (start 211 129.2) (end 211.1 129.1) (width 0.2) (layer "B.Cu") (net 3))
 (segment (start 214.7 113) (end 202.5 113) (width 0.2) (layer "B.Cu") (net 3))
 (segment (start 198.4 109.1) (end 198.1 109.4) (width 0.2) (layer "B.Cu") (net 3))
 (segment (start 222.4 135.2) (end 222.8898 134.7102) (width 0.2) (layer "B.Cu") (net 3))
 (segment (start 206.9 124) (end 206.9 124.9) (width 0.2) (layer "B.Cu") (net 3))
 (segment (start 214.8398 113.1398) (end 214.7 113) (width 0.2) (layer "B.Cu") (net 3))
 (segment (start 199.9 110.7) (end 199.1 111.5) (width 0.2) (layer "B.Cu") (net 3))
 (segment (start 210 128.2) (end 210 116.3) (width 0.2) (layer "B.Cu") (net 3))
 (segment (start 207.8 119.3) (end 207.6 119.1) (width 0.2) (layer "B.Cu") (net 3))
 (segment (start 217.7 112) (end 201 112) (width 0.2) (layer "B.Cu") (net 3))
 (segment (start 202.5 113) (end 201.9 113.6) (width 0.2) (layer "B.Cu") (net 3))
 (segment (start 206.8 123.9) (end 206.9 124) (width 0.2) (layer "B.Cu") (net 3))
 (segment (start 211.3 115.5) (end 211 115.2) (width 0.2) (layer "B.Cu") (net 3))
 (segment (start 200.4 133) (end 218.2 133) (width 0.2) (layer "B.Cu") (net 3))
 (segment (start 220.3 110.7) (end 199.9 110.7) (width 0.2) (layer "B.Cu") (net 3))
 (segment (start 241.665 109) (end 241.665 108.800001) (width 0.2) (layer "F.Cu") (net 11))
 (segment (start 247 110.5) (end 247 110.1) (width 0.2) (layer "F.Cu") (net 11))
 (segment (start 241.665 108.800001) (end 241.363999 108.499) (width 0.2) (layer "F.Cu") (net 11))
 (segment (start 204.599 120.8339) (end 204.599 125.6661) (width 0.2) (layer "F.Cu") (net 11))
 (segment (start 258.16 125.3) (end 258.16 123.76) (width 0.2) (layer "F.Cu") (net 11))
 (segment (start 245.1 109) (end 241.665 109) (width 0.2) (layer "F.Cu") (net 11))
 (segment (start 224.8298 128.635) (end 234.1048 137.91) (width 0.2) (layer "F.Cu") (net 11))
 (segment (start 204.599 125.6661) (end 207.5679 128.635) (width 0.2) (layer "F.Cu") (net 11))
 (segment (start 258.16 123.76) (end 257 122.6) (width 0.2) (layer "F.Cu") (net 11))
 (segment (start 263.24 125.3) (end 258.16 125.3) (width 0.2) (layer "F.Cu") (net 11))
 (segment (start 241.363999 108.499) (end 216.9339 108.499) (width 0.2) (layer "F.Cu") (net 11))
 (segment (start 245.5 108.6) (end 245.1 109) (width 0.2) (layer "F.Cu") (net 11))
 (segment (start 216.9339 108.499) (end 204.599 120.8339) (width 0.2) (layer "F.Cu") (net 11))
 (segment (start 207.5679 128.635) (end 224.8298 128.635) (width 0.2) (layer "F.Cu") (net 11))
 (segment (start 247 110.1) (end 245.5 108.6) (width 0.2) (layer "F.Cu") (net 11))
 (via (at 247 110.5) (size 0.6) (drill 0.3) (layers "F.Cu" "B.Cu") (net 11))
 (via (at 257 122.6) (size 0.6) (drill 0.3) (layers "F.Cu" "B.Cu") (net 11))
 (segment (start 253.912621 122.6) (end 244.2 112.887379) (width 0.2) (layer "B.Cu") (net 11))
 (segment (start 244.2 112.887379) (end 244.2 109.6) (width 0.2) (layer "B.Cu") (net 11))
 (segment (start 244.2 109.6) (end 246.1 109.6) (width 0.2) (layer "B.Cu") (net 11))
 (segment (start 246.1 109.6) (end 247 110.5) (width 0.2) (layer "B.Cu") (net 11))
 (segment (start 257 122.6) (end 253.912621 122.6) (width 0.2) (layer "B.Cu") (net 11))
 (segment (start 216.3248 117.59) (end 212.5 113.7652) (width 0.2) (layer "F.Cu") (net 1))
 (segment (start 205 121) (end 205 125.5) (width 0.2) (layer "F.Cu") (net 1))
 (segment (start 251.5 113.5) (end 252.5 114.5) (width 0.2) (layer "F.Cu") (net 1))
 (segment (start 254.6 117.8) (end 254.6 120.5) (width 0.2) (layer "F.Cu") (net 1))
 (segment (start 263.24 117.2) (end 258.16 117.2) (width 0.2) (layer "F.Cu") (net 1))
 (segment (start 219.366796 113.5) (end 251.5 113.5) (width 0.2) (layer "F.Cu") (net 1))
 (segment (start 258.16 117.2) (end 258.16 120.24) (width 0.2) (layer "F.Cu") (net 1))
 (segment (start 252.5 114.5) (end 252.376 114.624) (width 0.2) (layer "F.Cu") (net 1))
 (segment (start 212.5 113.7652) (end 212.5 113.5) (width 0.2) (layer "F.Cu") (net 1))
 (segment (start 252.376 114.624) (end 252.376 118.276) (width 0.2) (layer "F.Cu") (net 1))
 (segment (start 207.366796 125.5) (end 219.366796 113.5) (width 0.2) (layer "F.Cu") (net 1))
 (segment (start 205 125.5) (end 207.366796 125.5) (width 0.2) (layer "F.Cu") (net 1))
 (segment (start 212.5 113.5) (end 205 121) (width 0.2) (layer "F.Cu") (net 1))
 (segment (start 252.376 118.276) (end 254.6 120.5) (width 0.2) (layer "F.Cu") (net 1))
 (segment (start 258.16 120.24) (end 257.8 120.6) (width 0.2) (layer "F.Cu") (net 1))
 (via (at 254.6 117.8) (size 0.6) (drill 0.3) (layers "F.Cu" "B.Cu") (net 1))
 (via (at 257.8 120.6) (size 0.6) (drill 0.3) (layers "F.Cu" "B.Cu") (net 1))
 (segment (start 257.4 120.6) (end 254.6 117.8) (width 0.2) (layer "B.Cu") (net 1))
 (segment (start 257.8 120.6) (end 257.4 120.6) (width 0.2) (layer "B.Cu") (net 1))
 (segment (start 258.16 131.26) (end 257.3 130.4) (width 0.2) (layer "F.Cu") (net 2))
 (segment (start 258.16 133.3) (end 258.16 131.26) (width 0.2) (layer "F.Cu") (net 2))
 (segment (start 263.24 133.3) (end 258.16 133.3) (width 0.2) (layer "F.Cu") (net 2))
 (via (at 257.3 130.4) (size 0.6) (drill 0.3) (layers "F.Cu" "B.Cu") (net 2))
 (segment (start 246.8048 119.9048) (end 246.8048 117.59) (width 0.2) (layer "B.Cu") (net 2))
 (segment (start 257.3 130.4) (end 246.8048 119.9048) (width 0.2) (layer "B.Cu") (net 2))
 (segment (start 235.46 109.95) (end 236.55 111.04) (width 0.2) (layer "F.Cu") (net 14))
 (segment (start 237.76 133.48) (end 236.55 134.69) (width 0.2) (layer "F.Cu") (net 14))
 (segment (start 232.49 109.95) (end 227.41 109.95) (width 0.2) (layer "F.Cu") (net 14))
 (segment (start 232.49 109.95) (end 235.46 109.95) (width 0.2) (layer "F.Cu") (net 14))
 (segment (start 237.76 128.1) (end 237.76 133.48) (width 0.2) (layer "F.Cu") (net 14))
 (segment (start 236.55 134.69) (end 238.5048 134.69) (width 0.2) (layer "F.Cu") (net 14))
 (segment (start 238.5048 134.69) (end 241.7248 137.91) (width 0.2) (layer "F.Cu") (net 14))
 (via (at 236.55 111.04) (size 0.6) (drill 0.3) (layers "F.Cu" "B.Cu") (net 14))
 (via (at 237.76 128.1) (size 0.6) (drill 0.3) (layers "F.Cu" "B.Cu") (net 14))
 (segment (start 237.76 112.25) (end 237.76 128.1) (width 0.2) (layer "B.Cu") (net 14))
 (segment (start 236.55 111.04) (end 237.76 112.25) (width 0.2) (layer "B.Cu") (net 14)))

